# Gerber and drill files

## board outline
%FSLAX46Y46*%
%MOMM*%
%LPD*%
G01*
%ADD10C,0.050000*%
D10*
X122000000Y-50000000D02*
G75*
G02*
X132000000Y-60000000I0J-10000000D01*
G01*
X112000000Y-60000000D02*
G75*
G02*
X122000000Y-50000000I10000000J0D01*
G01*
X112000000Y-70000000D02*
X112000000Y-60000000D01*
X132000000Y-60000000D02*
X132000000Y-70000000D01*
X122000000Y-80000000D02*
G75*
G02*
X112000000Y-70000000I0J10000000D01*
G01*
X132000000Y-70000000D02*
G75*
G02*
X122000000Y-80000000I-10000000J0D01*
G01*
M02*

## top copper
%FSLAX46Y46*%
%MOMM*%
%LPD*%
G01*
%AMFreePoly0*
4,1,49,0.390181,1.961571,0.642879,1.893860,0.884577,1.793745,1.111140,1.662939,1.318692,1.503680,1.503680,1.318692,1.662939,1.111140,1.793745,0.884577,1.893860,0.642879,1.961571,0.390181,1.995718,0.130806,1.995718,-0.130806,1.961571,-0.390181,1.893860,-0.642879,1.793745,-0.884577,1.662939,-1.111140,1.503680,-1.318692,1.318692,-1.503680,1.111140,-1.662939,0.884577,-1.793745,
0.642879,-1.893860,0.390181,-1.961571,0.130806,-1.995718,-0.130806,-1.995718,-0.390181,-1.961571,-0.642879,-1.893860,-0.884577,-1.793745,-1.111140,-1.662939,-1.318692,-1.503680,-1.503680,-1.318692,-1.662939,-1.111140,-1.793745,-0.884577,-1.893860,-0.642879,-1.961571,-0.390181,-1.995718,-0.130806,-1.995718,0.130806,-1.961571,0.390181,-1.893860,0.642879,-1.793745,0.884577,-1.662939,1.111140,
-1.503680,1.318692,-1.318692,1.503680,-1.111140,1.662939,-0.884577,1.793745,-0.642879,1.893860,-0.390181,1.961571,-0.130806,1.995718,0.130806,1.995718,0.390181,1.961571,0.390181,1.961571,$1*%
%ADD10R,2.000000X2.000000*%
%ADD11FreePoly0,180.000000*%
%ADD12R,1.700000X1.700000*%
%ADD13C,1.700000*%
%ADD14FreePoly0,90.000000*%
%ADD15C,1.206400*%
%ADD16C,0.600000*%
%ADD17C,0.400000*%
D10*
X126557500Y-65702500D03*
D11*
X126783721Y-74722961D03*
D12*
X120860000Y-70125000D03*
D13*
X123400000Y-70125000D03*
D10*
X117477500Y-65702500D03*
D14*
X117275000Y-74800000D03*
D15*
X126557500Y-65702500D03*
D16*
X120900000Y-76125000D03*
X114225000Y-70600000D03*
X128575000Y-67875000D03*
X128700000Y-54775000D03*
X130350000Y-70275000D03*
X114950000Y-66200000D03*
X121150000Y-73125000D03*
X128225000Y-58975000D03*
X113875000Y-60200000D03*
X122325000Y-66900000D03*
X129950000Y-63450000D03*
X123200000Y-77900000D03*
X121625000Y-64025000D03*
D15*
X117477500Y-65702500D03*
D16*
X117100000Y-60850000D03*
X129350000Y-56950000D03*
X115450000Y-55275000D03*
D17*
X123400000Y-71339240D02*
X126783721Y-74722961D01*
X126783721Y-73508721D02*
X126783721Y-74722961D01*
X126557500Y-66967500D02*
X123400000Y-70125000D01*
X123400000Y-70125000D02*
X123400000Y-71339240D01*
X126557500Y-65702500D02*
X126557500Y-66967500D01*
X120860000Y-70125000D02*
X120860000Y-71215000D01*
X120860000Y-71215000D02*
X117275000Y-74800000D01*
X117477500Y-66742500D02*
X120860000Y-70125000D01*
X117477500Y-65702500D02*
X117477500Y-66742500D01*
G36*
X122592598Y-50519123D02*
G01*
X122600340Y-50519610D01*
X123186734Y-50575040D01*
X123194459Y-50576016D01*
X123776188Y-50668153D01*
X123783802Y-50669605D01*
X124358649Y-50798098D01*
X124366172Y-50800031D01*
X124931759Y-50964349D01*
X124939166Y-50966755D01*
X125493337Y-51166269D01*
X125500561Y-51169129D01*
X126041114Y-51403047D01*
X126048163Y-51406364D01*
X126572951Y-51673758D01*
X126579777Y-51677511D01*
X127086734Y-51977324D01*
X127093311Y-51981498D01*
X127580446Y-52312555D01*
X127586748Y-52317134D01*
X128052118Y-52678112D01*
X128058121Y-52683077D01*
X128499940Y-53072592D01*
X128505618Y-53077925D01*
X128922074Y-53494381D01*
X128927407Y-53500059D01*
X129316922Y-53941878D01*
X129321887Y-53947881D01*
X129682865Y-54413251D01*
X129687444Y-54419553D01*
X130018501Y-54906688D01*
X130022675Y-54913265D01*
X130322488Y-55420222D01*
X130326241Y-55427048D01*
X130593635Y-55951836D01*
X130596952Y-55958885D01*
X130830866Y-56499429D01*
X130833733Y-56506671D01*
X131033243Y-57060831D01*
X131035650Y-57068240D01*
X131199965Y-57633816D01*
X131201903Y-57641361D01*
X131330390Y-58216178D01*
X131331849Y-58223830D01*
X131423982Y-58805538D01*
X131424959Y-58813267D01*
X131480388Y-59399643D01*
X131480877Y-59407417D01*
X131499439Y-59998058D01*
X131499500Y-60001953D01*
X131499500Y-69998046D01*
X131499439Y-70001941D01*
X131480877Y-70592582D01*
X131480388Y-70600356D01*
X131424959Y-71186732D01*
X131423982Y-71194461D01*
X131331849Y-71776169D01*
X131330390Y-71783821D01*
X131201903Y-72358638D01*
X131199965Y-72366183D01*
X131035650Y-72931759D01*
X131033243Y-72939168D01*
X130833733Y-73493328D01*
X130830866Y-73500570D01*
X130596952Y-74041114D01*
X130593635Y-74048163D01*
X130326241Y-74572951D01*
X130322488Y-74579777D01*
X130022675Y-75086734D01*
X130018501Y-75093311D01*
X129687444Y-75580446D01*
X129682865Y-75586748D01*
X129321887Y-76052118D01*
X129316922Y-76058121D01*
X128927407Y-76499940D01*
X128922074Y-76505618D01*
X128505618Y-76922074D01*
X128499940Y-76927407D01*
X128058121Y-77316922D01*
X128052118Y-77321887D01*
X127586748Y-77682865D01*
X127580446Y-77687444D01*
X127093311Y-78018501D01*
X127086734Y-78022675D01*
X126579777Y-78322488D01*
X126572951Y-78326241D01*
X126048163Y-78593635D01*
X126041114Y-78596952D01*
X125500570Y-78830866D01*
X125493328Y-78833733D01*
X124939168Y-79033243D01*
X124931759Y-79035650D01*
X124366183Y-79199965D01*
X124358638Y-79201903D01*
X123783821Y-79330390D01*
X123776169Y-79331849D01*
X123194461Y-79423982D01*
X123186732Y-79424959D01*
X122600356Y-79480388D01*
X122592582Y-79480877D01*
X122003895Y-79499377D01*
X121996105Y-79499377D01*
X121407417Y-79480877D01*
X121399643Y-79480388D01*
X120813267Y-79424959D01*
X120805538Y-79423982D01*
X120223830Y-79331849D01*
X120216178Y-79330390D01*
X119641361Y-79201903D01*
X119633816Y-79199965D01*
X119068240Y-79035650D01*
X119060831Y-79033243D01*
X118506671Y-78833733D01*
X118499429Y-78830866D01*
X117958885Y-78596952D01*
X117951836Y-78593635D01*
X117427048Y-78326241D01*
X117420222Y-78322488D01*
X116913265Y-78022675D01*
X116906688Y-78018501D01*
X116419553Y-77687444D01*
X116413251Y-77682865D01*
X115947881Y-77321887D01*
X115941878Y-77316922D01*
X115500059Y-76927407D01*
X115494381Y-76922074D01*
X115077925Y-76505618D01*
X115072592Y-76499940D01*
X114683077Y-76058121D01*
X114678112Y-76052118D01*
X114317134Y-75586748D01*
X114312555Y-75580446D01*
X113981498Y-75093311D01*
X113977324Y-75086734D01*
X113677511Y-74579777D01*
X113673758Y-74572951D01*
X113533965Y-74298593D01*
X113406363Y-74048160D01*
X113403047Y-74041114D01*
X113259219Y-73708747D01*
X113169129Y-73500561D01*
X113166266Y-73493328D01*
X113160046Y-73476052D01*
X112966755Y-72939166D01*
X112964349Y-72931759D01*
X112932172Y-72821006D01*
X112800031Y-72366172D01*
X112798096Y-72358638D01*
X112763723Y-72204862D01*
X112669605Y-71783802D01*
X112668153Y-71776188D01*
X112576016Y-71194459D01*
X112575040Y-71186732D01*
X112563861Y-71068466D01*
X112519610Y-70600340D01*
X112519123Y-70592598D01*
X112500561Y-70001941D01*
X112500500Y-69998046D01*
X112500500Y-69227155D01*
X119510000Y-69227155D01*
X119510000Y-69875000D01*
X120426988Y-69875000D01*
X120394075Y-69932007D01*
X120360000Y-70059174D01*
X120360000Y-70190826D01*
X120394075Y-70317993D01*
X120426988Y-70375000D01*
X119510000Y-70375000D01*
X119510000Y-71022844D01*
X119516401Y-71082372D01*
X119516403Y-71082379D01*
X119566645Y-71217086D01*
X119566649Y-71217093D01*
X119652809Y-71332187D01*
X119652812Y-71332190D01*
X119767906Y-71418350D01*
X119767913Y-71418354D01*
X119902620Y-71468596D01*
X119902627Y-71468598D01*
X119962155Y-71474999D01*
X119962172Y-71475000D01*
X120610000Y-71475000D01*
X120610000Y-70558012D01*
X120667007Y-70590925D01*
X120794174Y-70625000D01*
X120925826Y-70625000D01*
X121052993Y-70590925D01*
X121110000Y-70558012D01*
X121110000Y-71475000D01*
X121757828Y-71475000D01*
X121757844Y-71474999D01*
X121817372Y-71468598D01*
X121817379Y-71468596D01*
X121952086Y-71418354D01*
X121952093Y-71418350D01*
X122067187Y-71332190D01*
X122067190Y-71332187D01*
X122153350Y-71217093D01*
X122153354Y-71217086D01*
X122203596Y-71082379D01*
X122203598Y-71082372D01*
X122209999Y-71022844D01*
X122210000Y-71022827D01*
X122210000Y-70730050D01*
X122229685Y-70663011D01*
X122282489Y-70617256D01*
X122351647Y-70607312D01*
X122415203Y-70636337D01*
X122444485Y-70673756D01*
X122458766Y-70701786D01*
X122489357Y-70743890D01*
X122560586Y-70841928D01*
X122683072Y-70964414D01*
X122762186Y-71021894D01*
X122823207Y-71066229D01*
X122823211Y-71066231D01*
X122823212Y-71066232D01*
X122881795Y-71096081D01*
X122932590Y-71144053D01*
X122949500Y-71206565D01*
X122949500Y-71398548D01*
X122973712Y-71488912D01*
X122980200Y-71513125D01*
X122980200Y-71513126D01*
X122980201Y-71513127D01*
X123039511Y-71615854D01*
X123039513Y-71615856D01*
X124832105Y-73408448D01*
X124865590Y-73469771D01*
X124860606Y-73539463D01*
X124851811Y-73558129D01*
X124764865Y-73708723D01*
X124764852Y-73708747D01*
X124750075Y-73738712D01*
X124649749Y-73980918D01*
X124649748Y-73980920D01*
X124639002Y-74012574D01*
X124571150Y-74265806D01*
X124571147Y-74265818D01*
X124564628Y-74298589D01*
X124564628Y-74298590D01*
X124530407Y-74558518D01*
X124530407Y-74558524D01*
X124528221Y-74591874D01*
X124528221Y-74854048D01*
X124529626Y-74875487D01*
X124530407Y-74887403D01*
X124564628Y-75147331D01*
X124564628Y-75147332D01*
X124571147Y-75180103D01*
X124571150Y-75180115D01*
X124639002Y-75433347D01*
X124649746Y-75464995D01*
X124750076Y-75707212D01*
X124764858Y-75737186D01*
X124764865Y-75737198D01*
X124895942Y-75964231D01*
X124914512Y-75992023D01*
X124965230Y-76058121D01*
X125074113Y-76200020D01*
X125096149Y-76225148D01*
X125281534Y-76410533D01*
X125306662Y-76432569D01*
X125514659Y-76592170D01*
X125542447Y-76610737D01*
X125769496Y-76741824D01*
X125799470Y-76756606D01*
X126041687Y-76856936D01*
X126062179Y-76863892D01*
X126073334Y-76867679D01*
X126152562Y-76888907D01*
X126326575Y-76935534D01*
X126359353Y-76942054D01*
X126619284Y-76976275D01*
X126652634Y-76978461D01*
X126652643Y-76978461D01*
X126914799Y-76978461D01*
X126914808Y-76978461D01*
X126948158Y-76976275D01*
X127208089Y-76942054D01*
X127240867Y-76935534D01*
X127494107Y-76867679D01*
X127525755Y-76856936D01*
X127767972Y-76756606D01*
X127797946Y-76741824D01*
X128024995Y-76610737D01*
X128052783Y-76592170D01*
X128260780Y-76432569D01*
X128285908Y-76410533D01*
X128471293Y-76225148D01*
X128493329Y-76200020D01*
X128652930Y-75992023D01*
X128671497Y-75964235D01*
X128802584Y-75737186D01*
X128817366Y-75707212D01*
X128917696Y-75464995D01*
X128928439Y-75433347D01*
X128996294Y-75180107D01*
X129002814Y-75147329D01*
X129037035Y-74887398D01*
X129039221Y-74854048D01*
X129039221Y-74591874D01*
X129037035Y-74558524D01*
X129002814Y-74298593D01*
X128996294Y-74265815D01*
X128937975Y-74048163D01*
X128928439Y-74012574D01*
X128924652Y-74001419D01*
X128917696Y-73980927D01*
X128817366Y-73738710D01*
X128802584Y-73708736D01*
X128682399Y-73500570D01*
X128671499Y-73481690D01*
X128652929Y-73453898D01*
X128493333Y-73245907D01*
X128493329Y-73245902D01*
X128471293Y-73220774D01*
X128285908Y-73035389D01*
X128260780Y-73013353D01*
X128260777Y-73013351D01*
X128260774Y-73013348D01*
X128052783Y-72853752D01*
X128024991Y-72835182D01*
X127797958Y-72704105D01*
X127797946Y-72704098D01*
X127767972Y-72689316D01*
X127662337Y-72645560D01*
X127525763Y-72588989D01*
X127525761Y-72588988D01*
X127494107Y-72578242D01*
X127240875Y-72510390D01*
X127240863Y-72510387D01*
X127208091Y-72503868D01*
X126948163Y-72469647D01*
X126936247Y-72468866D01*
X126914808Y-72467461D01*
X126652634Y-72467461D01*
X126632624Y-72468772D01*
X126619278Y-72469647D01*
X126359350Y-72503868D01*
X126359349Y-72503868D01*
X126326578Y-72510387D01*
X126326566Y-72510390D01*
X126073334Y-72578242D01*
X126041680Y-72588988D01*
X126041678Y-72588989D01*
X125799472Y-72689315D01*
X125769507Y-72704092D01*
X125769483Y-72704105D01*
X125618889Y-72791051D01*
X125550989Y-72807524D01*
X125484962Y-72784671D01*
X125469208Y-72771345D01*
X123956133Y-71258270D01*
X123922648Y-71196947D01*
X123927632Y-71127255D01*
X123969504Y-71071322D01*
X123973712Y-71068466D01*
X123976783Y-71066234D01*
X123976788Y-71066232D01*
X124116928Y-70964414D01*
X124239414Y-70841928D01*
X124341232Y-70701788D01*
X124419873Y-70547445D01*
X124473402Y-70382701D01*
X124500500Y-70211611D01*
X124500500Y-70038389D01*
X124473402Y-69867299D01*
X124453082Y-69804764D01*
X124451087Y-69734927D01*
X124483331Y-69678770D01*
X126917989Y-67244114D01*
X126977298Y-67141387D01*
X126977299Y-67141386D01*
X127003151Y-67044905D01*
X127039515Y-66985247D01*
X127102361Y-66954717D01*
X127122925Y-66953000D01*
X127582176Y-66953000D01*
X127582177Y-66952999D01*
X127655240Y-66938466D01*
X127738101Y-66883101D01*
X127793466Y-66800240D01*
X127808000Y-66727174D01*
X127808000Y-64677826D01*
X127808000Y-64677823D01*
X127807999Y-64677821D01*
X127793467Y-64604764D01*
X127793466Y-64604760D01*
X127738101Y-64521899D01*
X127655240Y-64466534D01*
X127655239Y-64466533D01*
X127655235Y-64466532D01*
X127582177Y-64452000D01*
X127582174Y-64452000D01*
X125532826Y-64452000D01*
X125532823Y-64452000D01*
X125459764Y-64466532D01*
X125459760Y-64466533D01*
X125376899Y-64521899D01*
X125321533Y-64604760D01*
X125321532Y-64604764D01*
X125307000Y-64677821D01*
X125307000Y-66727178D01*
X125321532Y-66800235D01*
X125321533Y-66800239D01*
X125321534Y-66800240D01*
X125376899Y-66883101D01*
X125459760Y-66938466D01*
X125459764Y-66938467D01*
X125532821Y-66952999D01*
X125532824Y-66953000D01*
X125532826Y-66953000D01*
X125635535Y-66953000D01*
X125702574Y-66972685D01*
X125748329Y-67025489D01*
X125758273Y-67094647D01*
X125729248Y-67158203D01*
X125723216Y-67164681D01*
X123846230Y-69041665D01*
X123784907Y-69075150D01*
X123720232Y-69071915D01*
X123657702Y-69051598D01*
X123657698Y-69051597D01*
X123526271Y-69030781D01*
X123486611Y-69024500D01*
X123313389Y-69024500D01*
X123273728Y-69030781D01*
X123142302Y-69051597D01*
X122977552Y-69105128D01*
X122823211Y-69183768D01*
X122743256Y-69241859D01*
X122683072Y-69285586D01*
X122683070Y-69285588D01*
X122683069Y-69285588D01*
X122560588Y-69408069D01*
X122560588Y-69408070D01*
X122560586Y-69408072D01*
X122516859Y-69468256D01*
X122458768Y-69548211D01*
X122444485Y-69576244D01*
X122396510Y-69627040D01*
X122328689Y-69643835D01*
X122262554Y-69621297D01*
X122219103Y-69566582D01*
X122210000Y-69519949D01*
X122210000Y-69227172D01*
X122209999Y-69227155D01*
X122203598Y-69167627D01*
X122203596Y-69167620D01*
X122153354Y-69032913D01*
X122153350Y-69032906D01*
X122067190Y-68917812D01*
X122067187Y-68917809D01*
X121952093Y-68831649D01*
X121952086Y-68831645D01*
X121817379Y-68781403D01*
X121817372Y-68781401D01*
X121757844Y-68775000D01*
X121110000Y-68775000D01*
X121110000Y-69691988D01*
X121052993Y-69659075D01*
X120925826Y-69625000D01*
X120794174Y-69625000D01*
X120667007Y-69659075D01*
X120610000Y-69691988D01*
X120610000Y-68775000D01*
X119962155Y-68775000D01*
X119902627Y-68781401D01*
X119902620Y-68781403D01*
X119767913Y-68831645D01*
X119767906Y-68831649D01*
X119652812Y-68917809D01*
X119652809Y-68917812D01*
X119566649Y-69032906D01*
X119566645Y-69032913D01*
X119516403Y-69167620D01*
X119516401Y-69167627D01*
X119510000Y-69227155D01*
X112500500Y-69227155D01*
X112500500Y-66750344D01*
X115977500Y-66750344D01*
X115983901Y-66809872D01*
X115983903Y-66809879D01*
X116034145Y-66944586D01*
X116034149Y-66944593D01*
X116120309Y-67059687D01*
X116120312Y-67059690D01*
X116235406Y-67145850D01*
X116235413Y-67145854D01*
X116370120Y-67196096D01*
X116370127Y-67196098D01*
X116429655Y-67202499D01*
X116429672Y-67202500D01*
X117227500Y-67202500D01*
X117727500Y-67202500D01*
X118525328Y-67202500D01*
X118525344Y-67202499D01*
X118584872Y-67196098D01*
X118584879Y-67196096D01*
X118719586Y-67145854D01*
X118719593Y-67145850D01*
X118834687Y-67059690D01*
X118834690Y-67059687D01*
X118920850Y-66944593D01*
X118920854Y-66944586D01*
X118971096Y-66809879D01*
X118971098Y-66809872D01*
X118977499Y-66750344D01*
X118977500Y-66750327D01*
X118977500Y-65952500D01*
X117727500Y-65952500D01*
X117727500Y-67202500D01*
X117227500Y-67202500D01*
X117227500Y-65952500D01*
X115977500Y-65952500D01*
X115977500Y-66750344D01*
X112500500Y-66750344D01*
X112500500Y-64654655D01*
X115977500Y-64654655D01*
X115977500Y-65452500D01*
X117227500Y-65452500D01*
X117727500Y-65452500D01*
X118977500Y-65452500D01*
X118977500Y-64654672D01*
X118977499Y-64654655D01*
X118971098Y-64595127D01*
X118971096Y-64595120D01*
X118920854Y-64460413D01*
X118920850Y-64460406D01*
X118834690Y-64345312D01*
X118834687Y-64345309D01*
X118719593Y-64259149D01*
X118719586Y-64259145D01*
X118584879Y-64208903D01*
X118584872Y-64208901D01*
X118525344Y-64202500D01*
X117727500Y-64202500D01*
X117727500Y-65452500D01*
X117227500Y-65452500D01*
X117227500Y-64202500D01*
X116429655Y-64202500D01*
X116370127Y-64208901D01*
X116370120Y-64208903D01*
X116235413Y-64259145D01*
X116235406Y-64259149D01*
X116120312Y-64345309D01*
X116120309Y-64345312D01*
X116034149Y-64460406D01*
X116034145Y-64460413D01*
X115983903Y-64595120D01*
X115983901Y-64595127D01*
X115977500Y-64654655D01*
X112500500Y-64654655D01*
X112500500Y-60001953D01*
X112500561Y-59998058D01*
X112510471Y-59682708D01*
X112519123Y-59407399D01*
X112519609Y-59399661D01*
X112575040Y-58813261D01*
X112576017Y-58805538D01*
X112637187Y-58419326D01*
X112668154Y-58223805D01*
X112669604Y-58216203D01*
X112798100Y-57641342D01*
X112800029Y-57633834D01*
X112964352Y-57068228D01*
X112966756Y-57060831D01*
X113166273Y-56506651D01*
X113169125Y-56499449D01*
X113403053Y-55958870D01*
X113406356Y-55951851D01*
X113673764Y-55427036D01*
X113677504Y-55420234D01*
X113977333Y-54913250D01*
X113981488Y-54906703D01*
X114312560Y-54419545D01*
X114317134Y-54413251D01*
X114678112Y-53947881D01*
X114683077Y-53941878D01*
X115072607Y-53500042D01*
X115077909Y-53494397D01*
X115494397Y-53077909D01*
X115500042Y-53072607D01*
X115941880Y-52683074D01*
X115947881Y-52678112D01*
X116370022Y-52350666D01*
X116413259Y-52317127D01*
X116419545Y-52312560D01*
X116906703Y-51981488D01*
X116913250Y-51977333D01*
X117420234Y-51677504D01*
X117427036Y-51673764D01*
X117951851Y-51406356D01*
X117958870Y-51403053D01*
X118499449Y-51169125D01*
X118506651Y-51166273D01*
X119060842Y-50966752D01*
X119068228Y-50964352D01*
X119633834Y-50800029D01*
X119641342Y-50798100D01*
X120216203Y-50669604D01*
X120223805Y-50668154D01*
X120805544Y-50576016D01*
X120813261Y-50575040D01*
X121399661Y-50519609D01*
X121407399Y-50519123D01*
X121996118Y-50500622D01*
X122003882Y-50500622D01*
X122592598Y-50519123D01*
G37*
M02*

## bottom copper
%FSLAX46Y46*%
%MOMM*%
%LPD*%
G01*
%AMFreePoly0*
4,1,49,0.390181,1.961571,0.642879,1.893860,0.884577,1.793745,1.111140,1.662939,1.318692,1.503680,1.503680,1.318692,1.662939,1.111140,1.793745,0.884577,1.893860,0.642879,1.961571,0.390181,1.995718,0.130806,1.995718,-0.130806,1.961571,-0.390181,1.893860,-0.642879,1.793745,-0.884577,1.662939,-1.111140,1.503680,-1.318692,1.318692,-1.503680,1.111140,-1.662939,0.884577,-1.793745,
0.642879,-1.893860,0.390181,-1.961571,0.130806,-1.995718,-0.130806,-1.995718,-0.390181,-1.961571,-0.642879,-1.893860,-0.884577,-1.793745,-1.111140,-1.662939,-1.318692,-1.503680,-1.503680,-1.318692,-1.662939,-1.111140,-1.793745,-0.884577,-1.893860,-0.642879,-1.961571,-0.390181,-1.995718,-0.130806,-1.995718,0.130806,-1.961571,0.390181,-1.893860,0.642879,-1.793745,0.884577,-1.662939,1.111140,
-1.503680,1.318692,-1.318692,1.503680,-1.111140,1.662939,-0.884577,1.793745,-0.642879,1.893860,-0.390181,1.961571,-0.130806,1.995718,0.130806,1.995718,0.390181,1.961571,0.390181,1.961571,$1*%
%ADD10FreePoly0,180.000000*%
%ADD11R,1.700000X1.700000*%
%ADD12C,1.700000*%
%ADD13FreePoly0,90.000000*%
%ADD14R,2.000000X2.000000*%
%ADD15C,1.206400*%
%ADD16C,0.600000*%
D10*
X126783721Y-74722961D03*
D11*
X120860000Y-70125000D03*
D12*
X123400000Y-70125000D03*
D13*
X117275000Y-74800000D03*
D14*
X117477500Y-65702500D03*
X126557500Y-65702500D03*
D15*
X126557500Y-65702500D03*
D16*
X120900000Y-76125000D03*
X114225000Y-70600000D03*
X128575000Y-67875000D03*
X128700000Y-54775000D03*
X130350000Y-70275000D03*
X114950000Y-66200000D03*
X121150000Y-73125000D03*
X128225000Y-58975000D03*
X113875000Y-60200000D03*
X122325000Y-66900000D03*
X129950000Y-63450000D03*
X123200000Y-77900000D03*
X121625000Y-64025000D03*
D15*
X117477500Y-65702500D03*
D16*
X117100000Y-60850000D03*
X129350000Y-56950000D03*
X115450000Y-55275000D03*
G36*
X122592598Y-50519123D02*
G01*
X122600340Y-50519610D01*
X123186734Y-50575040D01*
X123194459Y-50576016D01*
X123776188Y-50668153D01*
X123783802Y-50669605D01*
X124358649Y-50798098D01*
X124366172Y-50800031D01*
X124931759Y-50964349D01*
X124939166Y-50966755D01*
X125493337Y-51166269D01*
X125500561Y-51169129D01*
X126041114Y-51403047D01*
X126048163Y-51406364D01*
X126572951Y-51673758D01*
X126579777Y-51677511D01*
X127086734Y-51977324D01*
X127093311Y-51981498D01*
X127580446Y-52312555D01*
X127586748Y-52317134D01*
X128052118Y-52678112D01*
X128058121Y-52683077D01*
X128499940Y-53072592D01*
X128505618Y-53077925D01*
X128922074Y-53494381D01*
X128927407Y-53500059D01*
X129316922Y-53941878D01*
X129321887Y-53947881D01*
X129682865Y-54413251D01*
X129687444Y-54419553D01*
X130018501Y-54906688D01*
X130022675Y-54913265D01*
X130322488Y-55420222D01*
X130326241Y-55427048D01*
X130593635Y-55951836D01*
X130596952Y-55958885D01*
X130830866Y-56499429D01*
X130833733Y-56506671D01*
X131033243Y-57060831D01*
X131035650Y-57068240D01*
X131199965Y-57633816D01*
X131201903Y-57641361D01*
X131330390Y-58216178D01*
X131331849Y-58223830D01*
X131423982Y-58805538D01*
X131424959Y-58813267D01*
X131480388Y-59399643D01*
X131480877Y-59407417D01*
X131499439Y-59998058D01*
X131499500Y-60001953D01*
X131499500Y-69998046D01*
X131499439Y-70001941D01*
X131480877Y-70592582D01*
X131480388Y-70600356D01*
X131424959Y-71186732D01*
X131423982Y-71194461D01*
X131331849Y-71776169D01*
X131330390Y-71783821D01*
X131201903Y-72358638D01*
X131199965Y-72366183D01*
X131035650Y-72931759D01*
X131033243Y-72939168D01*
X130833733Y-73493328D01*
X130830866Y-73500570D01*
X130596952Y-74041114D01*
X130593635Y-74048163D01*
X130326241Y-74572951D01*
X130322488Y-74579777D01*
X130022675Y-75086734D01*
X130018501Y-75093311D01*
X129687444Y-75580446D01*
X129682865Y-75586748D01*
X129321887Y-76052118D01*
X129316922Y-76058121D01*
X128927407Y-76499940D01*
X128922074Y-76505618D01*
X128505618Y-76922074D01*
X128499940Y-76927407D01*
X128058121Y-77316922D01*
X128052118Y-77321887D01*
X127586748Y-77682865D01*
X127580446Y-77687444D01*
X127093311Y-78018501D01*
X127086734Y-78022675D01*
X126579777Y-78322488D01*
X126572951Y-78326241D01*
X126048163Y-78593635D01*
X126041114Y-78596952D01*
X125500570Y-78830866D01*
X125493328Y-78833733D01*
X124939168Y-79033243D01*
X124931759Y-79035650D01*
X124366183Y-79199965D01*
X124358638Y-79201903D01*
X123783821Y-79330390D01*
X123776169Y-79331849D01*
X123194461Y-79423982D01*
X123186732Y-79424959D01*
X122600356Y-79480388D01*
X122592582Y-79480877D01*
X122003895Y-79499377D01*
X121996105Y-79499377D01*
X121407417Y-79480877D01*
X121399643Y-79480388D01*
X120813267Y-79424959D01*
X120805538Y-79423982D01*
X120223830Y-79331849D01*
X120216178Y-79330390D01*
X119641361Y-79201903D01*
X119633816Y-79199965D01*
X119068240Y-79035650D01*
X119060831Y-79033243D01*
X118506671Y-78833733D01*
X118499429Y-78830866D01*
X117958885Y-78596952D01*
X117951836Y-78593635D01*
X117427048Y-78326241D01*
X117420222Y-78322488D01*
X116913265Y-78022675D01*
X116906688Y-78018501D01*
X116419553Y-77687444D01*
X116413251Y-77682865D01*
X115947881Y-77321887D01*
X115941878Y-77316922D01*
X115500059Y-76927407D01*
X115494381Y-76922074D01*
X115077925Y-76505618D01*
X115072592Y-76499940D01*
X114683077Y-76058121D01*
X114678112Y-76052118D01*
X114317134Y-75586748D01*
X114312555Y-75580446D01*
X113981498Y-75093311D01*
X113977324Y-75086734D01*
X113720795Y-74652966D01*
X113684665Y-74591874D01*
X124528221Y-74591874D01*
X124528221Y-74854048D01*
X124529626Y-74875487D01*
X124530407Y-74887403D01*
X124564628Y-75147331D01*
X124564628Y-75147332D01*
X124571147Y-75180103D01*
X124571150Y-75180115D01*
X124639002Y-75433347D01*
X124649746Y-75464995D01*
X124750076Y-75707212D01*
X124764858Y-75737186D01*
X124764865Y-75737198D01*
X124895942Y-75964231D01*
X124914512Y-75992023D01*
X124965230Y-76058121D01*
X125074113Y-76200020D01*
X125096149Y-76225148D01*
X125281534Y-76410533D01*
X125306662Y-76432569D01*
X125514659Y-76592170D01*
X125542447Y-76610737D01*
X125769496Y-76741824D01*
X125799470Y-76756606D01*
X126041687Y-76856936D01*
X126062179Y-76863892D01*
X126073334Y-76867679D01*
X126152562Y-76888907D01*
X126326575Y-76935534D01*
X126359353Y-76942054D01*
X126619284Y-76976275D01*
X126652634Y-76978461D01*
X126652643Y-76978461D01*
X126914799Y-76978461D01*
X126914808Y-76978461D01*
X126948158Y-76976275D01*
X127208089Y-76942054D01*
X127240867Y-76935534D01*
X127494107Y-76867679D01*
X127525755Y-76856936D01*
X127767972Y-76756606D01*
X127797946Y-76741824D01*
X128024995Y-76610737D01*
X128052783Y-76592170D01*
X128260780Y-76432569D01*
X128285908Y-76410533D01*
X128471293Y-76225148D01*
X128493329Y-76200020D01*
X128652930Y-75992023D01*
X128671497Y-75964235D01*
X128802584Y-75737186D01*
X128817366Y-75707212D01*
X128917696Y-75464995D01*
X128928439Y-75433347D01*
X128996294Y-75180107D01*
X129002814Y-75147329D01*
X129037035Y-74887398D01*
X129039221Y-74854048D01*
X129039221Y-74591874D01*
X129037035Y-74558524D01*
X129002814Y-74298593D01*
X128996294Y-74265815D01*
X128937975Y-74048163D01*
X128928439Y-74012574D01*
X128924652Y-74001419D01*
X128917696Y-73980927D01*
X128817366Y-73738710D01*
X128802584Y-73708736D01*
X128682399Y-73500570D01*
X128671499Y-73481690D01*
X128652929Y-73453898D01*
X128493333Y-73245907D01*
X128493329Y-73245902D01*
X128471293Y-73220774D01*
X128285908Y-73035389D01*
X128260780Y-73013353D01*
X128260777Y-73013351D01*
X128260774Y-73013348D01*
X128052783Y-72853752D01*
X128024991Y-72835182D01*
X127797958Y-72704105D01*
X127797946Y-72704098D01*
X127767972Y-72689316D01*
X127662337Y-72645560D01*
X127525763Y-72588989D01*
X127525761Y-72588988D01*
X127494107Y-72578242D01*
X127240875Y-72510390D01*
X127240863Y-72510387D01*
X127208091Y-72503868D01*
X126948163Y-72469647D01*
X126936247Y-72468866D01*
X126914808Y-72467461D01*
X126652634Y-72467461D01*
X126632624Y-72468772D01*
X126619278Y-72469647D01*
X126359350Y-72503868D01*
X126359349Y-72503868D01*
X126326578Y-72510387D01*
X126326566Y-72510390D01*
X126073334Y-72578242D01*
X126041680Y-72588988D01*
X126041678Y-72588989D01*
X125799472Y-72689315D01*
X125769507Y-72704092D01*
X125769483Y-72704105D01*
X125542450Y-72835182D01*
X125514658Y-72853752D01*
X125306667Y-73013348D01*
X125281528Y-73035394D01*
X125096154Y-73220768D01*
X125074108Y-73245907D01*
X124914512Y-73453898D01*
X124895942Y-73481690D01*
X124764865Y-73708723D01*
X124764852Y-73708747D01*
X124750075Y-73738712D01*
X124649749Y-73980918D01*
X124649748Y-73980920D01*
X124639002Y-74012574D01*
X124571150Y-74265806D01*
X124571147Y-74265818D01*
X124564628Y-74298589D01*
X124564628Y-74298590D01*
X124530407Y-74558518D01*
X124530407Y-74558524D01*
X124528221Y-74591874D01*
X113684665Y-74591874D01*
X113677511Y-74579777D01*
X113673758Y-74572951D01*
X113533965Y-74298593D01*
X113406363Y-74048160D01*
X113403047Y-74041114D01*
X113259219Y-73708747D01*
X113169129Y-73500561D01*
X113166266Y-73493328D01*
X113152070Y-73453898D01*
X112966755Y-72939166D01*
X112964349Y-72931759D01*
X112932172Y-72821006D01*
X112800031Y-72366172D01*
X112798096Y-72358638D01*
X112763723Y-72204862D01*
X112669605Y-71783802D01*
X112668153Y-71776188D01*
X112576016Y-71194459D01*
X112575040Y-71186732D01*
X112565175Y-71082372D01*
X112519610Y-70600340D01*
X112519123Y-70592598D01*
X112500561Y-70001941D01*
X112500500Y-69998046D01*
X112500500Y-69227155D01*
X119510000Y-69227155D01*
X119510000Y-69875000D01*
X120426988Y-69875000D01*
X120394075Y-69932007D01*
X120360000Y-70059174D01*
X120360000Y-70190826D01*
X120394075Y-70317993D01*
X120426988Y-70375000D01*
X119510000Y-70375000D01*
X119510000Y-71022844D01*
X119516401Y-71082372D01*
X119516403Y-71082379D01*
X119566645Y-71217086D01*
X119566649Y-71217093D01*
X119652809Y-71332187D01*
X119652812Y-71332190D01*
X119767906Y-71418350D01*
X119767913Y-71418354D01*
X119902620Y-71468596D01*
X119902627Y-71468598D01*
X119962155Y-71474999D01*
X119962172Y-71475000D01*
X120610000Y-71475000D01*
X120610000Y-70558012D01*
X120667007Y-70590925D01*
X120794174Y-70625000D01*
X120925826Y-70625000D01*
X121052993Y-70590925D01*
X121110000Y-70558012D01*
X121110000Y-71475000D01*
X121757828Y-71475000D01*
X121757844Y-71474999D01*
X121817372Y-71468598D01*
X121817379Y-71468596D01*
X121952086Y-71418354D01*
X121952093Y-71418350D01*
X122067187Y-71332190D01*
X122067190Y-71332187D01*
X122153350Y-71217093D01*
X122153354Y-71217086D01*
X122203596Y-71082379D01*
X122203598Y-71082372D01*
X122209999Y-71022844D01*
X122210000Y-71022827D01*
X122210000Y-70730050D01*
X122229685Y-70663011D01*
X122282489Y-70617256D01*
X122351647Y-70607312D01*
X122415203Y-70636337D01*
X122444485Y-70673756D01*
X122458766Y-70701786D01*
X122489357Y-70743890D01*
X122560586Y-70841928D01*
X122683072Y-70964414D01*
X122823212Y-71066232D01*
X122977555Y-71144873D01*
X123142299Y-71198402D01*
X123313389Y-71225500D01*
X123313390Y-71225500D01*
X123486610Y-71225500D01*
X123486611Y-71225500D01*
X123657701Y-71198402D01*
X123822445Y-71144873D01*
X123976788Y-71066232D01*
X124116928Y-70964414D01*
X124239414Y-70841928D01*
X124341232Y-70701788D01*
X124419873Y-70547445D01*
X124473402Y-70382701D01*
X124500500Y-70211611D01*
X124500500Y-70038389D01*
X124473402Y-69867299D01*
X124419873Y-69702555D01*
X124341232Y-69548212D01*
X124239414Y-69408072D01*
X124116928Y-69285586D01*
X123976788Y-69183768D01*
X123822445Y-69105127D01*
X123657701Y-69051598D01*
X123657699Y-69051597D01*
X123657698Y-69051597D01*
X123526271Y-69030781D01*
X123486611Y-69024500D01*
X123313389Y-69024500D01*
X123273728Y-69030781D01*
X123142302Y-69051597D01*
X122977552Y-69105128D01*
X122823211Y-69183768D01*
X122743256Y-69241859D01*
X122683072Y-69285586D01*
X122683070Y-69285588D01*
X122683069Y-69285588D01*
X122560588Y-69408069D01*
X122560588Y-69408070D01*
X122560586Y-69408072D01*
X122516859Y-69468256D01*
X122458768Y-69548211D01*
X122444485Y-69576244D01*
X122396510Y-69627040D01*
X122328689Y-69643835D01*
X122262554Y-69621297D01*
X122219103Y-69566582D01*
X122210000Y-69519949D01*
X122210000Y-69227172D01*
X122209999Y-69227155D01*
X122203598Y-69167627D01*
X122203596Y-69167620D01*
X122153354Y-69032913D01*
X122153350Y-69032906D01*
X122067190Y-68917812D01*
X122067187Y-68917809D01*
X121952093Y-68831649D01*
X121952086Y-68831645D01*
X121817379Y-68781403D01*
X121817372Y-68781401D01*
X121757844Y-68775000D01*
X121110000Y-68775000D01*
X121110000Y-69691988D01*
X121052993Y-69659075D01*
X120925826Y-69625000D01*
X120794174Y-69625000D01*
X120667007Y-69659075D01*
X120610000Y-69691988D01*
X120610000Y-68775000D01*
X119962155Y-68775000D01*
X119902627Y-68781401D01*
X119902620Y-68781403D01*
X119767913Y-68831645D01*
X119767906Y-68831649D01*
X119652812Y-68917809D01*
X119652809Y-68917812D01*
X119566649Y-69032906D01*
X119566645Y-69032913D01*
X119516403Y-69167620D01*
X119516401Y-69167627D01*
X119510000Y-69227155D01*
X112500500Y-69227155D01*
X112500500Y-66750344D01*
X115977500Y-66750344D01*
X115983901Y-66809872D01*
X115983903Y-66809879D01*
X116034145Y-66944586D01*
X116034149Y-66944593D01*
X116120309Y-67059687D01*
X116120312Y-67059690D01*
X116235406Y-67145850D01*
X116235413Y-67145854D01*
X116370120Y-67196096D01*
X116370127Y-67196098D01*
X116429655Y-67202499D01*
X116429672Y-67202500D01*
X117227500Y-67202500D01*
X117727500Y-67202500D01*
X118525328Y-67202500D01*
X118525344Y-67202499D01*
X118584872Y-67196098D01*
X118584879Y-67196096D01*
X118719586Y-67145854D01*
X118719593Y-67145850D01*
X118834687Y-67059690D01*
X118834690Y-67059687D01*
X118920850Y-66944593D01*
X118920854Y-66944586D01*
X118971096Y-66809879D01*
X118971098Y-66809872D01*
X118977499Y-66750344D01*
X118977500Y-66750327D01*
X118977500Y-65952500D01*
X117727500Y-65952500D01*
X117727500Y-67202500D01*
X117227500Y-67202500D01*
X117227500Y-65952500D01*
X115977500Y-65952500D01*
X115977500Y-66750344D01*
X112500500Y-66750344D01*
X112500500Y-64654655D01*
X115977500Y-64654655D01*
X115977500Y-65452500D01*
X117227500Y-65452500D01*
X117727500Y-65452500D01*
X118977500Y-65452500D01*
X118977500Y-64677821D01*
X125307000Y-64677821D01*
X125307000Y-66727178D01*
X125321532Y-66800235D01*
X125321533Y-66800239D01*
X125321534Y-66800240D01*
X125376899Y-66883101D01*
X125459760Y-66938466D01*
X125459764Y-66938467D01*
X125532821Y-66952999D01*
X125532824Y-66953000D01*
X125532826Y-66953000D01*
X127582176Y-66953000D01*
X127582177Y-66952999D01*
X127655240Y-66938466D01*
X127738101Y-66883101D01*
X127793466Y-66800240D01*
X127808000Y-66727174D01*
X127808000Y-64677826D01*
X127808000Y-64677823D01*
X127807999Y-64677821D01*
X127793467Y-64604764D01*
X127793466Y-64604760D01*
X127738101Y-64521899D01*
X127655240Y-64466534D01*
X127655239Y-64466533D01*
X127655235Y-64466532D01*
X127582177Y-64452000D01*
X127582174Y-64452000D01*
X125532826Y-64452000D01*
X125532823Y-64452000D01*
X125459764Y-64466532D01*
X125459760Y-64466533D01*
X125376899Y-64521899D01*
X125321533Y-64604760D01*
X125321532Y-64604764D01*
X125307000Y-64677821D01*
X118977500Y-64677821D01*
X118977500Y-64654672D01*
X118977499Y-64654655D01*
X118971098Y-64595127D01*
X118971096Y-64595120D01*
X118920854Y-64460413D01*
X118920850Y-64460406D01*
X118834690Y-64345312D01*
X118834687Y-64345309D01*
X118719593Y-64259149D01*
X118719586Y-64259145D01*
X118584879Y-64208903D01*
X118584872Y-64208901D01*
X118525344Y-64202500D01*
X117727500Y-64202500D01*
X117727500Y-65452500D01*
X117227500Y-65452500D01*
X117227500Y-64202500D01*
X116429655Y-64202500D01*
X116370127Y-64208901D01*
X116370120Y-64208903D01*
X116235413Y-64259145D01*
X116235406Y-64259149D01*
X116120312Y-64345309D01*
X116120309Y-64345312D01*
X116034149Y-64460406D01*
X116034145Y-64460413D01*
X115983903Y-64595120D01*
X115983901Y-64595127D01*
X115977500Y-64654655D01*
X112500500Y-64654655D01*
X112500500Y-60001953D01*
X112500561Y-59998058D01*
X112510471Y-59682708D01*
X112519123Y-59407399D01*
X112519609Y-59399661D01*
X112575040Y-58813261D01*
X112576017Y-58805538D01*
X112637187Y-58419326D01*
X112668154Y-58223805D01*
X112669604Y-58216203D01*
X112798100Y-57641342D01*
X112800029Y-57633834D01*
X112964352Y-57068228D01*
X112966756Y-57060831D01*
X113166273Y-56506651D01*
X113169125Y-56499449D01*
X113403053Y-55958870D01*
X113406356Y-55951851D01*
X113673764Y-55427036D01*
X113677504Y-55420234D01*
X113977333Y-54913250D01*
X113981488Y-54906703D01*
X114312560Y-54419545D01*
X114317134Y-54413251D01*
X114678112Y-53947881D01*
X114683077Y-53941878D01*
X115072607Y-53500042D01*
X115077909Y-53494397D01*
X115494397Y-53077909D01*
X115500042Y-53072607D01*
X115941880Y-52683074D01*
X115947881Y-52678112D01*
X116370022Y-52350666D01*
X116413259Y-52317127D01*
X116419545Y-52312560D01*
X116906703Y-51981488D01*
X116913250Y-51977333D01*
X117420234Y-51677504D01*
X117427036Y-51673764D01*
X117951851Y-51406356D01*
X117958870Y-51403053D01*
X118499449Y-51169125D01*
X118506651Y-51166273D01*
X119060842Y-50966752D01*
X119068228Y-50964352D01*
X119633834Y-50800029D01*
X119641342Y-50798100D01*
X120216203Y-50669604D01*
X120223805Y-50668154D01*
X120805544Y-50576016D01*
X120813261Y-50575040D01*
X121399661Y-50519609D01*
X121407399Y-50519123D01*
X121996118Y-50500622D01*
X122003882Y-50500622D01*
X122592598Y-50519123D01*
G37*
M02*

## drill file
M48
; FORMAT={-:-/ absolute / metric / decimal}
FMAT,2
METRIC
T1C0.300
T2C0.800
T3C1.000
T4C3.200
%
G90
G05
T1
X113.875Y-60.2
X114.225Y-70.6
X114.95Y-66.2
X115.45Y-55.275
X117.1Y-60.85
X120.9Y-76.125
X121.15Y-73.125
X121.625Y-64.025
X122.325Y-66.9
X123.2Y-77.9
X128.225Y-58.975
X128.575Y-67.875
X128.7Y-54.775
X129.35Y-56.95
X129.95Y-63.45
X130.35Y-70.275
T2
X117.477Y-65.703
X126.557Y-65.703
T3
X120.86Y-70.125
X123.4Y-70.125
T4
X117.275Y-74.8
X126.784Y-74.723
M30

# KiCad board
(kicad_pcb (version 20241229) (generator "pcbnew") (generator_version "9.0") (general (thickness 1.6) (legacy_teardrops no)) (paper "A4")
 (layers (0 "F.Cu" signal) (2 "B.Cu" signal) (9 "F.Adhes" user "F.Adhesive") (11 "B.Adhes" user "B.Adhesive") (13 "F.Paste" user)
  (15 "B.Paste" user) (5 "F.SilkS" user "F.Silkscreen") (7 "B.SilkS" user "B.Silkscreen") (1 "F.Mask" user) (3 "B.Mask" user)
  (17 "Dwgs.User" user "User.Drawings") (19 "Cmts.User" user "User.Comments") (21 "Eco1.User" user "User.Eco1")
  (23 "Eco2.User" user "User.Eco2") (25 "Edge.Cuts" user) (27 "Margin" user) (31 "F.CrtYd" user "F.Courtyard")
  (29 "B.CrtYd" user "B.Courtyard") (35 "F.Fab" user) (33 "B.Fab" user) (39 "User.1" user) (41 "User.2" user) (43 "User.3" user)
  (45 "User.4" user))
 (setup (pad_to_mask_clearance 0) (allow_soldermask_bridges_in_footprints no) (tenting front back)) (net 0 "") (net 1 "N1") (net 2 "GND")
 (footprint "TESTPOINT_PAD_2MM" (layer "F.Cu") (at 126.5575 65.7025)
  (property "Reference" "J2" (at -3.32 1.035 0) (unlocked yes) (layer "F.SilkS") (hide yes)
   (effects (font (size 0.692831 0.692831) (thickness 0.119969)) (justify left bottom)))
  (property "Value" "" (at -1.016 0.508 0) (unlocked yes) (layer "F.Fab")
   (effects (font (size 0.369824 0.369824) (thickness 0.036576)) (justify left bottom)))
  (pad "Pin_2" smd rect (at 0 0) (size 2 2) (layers "F.Cu" "F.Mask") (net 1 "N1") (solder_mask_margin 0.0508) (solder_paste_margin 0)
   (thermal_bridge_angle 0)))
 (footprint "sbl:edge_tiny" (layer "F.Cu") (at 126.783721 74.722961 180)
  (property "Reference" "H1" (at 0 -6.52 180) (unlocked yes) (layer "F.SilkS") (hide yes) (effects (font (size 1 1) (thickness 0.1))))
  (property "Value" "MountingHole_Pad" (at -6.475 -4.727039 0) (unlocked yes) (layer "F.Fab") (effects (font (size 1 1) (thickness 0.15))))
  (pad "1" thru_hole custom (at 0 0 180) (size 4 4) (drill 3.2) (layers "*.Cu" "*.Mask") (remove_unused_layers no) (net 1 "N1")
   (options (clearance outline) (anchor circle)) (primitives)))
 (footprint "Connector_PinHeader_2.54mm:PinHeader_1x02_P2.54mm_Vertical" (layer "F.Cu") (at 120.86 70.125 90)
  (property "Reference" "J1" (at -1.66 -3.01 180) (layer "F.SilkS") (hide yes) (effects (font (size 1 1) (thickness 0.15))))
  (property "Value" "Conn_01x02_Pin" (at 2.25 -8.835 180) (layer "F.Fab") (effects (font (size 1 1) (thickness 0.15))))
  (pad "1" thru_hole rect (at 0 0 90) (size 1.7 1.7) (drill 1) (layers "*.Cu" "*.Mask") (remove_unused_layers no) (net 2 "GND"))
  (pad "2" thru_hole circle (at 0 2.54 90) (size 1.7 1.7) (drill 1) (layers "*.Cu" "*.Mask") (remove_unused_layers no) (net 1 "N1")))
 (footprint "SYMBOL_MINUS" (layer "F.Cu") (at 117.4775 68.1155)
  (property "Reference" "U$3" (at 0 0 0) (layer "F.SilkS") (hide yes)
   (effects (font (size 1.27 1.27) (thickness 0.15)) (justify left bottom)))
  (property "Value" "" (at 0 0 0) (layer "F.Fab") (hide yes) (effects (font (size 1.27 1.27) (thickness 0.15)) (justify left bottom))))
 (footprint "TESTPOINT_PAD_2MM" (layer "F.Cu") (at 117.4775 65.7025)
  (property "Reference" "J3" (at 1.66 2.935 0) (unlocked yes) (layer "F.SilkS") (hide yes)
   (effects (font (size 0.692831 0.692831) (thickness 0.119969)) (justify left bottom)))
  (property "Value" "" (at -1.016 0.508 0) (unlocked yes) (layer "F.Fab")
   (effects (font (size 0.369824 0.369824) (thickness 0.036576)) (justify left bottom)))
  (pad "Pin_1" smd rect (at 0 0) (size 2 2) (layers "F.Cu" "F.Mask") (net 2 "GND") (solder_mask_margin 0.0508) (solder_paste_margin 0)
   (thermal_bridge_angle 0)))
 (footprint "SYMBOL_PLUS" (layer "F.Cu") (at 126.5575 68.1155)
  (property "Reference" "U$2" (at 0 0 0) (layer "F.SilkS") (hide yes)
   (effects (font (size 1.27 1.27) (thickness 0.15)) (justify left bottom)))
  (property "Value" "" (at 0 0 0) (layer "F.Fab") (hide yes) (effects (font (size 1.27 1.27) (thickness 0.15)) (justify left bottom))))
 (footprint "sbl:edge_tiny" (layer "F.Cu") (at 117.275 74.8 90)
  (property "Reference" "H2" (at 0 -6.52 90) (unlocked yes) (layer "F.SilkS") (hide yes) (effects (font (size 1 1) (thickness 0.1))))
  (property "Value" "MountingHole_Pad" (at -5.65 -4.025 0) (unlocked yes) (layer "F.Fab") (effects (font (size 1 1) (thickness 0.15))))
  (pad "1" thru_hole custom (at 0 0 90) (size 4 4) (drill 3.2) (layers "*.Cu" "*.Mask") (remove_unused_layers no) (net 2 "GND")
   (zone_connect 2) (options (clearance outline) (anchor circle)) (primitives)))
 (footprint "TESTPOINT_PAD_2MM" (layer "B.Cu") (at 117.4775 65.7025 180)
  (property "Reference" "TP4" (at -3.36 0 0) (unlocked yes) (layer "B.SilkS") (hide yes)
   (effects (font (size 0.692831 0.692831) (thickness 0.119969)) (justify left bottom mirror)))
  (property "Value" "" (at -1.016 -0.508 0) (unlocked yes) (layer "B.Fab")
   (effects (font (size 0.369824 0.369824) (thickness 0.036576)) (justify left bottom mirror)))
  (pad "Pin_1" smd rect (at 0 0 180) (size 2 2) (layers "B.Cu" "B.Mask") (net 2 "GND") (solder_mask_margin 0.0508) (solder_paste_margin 0)
   (thermal_bridge_angle 0)))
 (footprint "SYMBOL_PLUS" (layer "B.Cu") (at 126.5575 68.1155)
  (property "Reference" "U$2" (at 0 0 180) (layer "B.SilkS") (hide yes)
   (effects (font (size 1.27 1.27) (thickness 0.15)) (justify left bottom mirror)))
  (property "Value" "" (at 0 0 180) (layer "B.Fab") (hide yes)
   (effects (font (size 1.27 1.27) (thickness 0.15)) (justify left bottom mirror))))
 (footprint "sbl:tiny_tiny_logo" (layer "B.Cu") (at 121.9375 56.5375 180)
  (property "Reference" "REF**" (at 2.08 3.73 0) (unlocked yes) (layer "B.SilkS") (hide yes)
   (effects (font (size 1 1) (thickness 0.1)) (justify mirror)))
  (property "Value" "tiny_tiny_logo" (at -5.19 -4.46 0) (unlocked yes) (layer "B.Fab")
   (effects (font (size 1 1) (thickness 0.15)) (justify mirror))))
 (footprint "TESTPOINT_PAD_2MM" (layer "B.Cu") (at 126.5575 65.7025 180)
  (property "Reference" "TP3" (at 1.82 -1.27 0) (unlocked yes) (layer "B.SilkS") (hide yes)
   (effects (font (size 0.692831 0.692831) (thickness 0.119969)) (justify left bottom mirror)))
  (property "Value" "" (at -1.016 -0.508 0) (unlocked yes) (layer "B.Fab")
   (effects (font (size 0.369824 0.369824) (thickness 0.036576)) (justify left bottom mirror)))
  (pad "1" smd rect (at 0 0 180) (size 2 2) (layers "B.Cu" "B.Mask") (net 1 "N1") (solder_mask_margin 0.0508) (solder_paste_margin 0)
   (thermal_bridge_angle 0)))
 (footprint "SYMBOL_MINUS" (layer "B.Cu") (at 117.4775 68.1155)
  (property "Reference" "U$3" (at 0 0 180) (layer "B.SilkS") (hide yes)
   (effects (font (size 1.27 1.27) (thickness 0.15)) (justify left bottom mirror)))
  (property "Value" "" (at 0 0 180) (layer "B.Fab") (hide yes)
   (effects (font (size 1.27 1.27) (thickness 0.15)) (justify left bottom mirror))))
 (gr_arc (start 122 50) (mid 129.071068 52.928932) (end 132 60) (stroke (width 0.05) (type default)) (layer "Edge.Cuts"))
 (gr_arc (start 112 60) (mid 114.928932 52.928932) (end 122 50) (stroke (width 0.05) (type default)) (layer "Edge.Cuts"))
 (gr_line (start 112 70) (end 112 60) (stroke (width 0.05) (type default)) (layer "Edge.Cuts"))
 (gr_line (start 132 60) (end 132 70) (stroke (width 0.05) (type default)) (layer "Edge.Cuts"))
 (gr_arc (start 122 80) (mid 114.928932 77.071068) (end 112 70) (stroke (width 0.05) (type default)) (layer "Edge.Cuts"))
 (gr_arc (start 132 70) (mid 129.071068 77.071068) (end 122 80) (stroke (width 0.05) (type default)) (layer "Edge.Cuts"))
 (segment (start 123.4 71.33924) (end 126.783721 74.722961) (width 0.4) (layer "F.Cu") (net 1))
 (segment (start 126.783721 73.508721) (end 126.783721 74.722961) (width 0.4) (layer "F.Cu") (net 1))
 (segment (start 126.5575 66.9675) (end 123.4 70.125) (width 0.4) (layer "F.Cu") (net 1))
 (segment (start 123.4 70.125) (end 123.4 71.33924) (width 0.4) (layer "F.Cu") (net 1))
 (segment (start 126.5575 65.7025) (end 126.5575 66.9675) (width 0.4) (layer "F.Cu") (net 1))
 (via (at 126.5575 65.7025) (size 1.2064) (drill 0.8) (layers "F.Cu" "B.Cu") (free yes) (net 1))
 (segment (start 120.86 70.125) (end 120.86 71.215) (width 0.4) (layer "F.Cu") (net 2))
 (segment (start 120.86 71.215) (end 117.275 74.8) (width 0.4) (layer "F.Cu") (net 2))
 (segment (start 117.4775 66.7425) (end 120.86 70.125) (width 0.4) (layer "F.Cu") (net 2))
 (segment (start 117.4775 65.7025) (end 117.4775 66.7425) (width 0.4) (layer "F.Cu") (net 2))
 (via (at 120.9 76.125) (size 0.6) (drill 0.3) (layers "F.Cu" "B.Cu") (free yes) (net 2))
 (via (at 114.225 70.6) (size 0.6) (drill 0.3) (layers "F.Cu" "B.Cu") (free yes) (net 2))
 (via (at 128.575 67.875) (size 0.6) (drill 0.3) (layers "F.Cu" "B.Cu") (free yes) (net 2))
 (via (at 128.7 54.775) (size 0.6) (drill 0.3) (layers "F.Cu" "B.Cu") (free yes) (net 2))
 (via (at 130.35 70.275) (size 0.6) (drill 0.3) (layers "F.Cu" "B.Cu") (free yes) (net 2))
 (via (at 114.95 66.2) (size 0.6) (drill 0.3) (layers "F.Cu" "B.Cu") (free yes) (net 2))
 (via (at 121.15 73.125) (size 0.6) (drill 0.3) (layers "F.Cu" "B.Cu") (free yes) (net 2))
 (via (at 128.225 58.975) (size 0.6) (drill 0.3) (layers "F.Cu" "B.Cu") (free yes) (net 2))
 (via (at 113.875 60.2) (size 0.6) (drill 0.3) (layers "F.Cu" "B.Cu") (free yes) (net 2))
 (via (at 122.325 66.9) (size 0.6) (drill 0.3) (layers "F.Cu" "B.Cu") (free yes) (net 2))
 (via (at 129.95 63.45) (size 0.6) (drill 0.3) (layers "F.Cu" "B.Cu") (free yes) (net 2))
 (via (at 123.2 77.9) (size 0.6) (drill 0.3) (layers "F.Cu" "B.Cu") (free yes) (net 2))
 (via (at 121.625 64.025) (size 0.6) (drill 0.3) (layers "F.Cu" "B.Cu") (free yes) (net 2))
 (via (at 117.4775 65.7025) (size 1.2064) (drill 0.8) (layers "F.Cu" "B.Cu") (free yes) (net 2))
 (via (at 117.1 60.85) (size 0.6) (drill 0.3) (layers "F.Cu" "B.Cu") (free yes) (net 2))
 (via (at 129.35 56.95) (size 0.6) (drill 0.3) (layers "F.Cu" "B.Cu") (free yes) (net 2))
 (via (at 115.45 55.275) (size 0.6) (drill 0.3) (layers "F.Cu" "B.Cu") (free yes) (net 2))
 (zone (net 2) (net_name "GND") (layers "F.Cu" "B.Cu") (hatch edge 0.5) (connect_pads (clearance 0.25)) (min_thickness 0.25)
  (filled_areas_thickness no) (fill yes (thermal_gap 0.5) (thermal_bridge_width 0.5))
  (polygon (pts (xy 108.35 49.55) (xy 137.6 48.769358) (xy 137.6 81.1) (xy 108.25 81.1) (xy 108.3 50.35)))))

